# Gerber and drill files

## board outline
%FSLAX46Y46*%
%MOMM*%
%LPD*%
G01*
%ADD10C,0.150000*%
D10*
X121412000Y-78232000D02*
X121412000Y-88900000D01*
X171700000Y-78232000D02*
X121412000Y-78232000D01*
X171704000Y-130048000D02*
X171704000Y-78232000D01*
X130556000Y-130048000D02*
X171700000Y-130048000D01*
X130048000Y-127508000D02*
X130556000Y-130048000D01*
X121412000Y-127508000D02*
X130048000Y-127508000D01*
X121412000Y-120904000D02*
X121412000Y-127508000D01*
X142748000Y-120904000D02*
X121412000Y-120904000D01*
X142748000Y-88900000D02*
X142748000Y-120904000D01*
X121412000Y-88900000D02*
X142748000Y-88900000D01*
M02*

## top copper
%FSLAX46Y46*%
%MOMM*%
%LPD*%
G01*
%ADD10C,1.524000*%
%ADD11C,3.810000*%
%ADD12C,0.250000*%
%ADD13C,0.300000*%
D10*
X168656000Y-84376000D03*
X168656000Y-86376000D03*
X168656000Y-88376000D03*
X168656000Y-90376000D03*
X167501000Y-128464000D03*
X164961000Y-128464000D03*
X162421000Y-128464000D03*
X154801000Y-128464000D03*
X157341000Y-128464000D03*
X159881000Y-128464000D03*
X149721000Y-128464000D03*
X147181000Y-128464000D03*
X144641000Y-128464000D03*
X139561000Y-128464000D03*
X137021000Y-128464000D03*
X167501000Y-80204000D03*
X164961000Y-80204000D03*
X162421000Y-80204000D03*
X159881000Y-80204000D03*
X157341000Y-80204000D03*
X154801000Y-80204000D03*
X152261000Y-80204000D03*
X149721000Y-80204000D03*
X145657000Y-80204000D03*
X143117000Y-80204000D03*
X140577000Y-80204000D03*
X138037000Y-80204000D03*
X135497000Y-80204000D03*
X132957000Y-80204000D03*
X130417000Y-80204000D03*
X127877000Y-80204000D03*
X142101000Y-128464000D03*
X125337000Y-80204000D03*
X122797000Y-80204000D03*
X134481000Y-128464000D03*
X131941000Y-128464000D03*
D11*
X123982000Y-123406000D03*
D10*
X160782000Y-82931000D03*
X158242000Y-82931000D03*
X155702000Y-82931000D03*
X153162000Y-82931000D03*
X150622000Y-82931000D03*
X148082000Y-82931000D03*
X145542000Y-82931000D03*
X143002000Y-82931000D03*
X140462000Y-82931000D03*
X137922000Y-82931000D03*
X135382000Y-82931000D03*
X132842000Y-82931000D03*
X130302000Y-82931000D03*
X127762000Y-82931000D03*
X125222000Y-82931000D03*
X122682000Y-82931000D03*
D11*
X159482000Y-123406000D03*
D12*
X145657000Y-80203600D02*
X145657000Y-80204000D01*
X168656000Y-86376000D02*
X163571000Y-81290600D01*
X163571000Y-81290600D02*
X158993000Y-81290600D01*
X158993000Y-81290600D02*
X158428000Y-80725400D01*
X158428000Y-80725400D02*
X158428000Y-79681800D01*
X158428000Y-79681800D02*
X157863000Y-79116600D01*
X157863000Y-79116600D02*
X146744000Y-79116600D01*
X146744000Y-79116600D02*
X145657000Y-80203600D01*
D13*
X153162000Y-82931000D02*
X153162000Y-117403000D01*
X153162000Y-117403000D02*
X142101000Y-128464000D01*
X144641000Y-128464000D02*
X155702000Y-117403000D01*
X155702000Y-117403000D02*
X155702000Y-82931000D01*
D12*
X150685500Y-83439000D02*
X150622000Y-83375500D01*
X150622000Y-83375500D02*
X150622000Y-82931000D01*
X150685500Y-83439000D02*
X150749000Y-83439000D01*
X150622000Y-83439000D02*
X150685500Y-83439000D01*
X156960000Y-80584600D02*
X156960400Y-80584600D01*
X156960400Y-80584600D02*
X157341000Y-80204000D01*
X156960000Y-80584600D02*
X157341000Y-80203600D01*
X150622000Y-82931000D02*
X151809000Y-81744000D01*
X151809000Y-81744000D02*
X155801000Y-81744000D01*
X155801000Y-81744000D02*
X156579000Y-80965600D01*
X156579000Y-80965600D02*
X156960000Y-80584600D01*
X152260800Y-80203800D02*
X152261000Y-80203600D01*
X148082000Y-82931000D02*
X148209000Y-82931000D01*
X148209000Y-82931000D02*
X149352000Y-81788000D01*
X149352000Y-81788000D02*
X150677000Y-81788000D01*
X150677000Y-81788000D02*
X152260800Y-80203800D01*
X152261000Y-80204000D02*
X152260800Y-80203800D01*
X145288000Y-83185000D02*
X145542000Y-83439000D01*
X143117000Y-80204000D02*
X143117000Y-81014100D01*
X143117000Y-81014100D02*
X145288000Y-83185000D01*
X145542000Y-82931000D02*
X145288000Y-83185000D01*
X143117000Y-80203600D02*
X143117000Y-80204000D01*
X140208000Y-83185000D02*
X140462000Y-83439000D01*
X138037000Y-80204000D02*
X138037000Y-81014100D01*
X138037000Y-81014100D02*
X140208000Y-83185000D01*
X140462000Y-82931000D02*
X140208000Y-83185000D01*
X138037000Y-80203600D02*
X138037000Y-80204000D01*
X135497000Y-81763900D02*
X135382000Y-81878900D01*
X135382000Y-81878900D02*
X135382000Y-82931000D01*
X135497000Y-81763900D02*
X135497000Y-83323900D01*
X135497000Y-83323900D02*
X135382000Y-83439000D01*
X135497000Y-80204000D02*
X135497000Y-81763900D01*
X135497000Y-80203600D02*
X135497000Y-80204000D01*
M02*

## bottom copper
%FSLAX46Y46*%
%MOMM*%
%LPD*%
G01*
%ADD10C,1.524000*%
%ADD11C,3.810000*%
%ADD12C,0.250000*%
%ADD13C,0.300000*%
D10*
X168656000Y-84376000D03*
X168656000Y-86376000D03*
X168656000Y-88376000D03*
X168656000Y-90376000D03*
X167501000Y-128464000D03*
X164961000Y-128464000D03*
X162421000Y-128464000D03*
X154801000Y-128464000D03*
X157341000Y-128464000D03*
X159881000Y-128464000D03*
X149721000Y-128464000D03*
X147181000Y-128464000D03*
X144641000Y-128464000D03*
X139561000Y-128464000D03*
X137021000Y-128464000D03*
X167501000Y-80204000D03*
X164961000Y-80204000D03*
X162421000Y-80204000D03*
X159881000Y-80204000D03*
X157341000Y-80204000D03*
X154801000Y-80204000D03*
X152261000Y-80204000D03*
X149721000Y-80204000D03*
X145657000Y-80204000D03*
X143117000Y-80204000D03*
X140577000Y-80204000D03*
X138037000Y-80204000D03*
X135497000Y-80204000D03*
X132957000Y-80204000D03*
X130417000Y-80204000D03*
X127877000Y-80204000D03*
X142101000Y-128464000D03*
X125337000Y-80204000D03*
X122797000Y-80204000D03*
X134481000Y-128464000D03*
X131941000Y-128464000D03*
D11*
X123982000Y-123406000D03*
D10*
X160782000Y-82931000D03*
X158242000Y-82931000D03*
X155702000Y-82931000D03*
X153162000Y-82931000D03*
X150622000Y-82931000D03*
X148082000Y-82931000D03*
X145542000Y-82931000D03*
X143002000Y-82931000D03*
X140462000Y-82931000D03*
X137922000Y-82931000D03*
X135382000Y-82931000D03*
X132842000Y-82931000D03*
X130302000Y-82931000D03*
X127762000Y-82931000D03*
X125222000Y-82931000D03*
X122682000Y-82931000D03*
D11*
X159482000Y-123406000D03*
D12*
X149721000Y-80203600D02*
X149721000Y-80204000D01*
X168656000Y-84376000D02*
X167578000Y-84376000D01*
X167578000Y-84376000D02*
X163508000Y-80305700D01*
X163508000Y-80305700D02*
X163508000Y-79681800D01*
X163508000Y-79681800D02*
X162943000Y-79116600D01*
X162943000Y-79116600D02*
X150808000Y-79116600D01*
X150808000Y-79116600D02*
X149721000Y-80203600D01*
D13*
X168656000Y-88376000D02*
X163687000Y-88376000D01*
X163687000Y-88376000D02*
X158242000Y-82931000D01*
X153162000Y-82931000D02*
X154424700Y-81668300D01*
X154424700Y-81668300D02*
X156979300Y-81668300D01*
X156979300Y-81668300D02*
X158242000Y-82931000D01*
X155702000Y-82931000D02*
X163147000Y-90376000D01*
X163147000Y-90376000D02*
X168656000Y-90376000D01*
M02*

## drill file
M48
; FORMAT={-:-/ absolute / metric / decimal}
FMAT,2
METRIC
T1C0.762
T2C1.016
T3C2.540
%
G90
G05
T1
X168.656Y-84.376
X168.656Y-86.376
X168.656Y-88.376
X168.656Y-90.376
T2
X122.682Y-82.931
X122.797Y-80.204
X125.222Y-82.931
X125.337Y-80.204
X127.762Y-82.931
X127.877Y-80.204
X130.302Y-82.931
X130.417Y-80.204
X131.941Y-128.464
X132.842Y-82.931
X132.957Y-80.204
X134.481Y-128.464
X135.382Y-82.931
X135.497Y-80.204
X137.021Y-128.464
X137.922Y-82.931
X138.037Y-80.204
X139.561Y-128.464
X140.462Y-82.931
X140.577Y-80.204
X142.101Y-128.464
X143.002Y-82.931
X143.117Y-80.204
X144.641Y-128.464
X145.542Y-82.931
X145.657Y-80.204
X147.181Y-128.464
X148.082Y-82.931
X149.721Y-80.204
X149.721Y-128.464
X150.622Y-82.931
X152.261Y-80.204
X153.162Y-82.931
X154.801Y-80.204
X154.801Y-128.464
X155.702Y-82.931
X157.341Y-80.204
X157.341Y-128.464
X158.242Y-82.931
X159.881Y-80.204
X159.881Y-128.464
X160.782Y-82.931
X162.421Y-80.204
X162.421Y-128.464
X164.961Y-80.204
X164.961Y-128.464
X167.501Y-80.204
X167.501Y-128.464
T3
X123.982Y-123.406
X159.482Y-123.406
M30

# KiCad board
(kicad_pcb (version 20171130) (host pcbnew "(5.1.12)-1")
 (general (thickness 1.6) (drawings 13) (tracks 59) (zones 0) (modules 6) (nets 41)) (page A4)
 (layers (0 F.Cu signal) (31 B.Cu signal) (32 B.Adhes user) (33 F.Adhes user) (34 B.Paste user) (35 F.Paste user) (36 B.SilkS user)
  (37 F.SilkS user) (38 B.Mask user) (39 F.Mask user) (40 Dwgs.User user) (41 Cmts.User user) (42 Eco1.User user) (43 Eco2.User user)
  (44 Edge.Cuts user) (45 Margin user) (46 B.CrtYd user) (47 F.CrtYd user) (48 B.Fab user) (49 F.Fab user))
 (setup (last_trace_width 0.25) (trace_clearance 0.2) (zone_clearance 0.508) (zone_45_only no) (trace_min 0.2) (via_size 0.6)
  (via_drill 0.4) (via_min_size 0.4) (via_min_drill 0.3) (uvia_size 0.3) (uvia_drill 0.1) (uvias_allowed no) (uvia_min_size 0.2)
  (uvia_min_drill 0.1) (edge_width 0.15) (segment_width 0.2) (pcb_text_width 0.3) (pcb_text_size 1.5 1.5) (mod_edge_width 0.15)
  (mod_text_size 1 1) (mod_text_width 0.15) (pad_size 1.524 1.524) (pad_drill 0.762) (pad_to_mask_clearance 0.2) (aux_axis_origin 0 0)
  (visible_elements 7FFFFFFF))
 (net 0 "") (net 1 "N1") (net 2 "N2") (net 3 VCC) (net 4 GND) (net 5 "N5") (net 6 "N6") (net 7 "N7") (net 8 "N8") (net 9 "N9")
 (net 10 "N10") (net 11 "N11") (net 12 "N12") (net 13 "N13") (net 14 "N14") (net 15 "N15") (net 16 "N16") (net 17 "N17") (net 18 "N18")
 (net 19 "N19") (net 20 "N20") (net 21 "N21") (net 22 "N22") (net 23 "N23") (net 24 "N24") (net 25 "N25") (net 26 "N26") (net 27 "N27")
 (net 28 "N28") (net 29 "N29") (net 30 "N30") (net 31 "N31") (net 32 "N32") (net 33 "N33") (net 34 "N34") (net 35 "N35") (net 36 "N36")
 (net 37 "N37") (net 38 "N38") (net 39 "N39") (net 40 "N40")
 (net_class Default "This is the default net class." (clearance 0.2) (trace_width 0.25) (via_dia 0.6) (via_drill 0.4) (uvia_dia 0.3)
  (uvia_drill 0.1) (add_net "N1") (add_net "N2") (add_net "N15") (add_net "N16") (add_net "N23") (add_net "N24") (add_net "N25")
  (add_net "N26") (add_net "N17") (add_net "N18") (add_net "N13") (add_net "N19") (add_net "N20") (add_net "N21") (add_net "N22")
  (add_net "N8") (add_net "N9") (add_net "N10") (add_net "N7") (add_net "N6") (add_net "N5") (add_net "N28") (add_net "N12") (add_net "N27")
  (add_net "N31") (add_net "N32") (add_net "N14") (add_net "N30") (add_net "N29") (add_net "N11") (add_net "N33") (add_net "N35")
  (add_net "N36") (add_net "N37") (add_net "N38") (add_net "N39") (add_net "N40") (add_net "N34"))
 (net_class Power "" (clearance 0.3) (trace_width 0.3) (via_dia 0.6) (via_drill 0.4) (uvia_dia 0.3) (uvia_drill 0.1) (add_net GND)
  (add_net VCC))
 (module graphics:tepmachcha (layer B.Cu) (at 166.624 113.665 90)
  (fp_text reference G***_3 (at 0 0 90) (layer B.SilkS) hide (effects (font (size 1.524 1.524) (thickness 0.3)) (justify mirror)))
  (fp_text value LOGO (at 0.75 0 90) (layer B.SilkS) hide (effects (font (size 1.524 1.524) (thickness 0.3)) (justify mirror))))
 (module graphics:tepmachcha (layer F.Cu) (at 167.386 100.33 270)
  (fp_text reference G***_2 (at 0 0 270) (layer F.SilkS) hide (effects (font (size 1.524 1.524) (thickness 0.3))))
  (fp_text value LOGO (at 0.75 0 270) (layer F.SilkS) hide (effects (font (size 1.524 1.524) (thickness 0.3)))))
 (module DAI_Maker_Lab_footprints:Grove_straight (layer F.Cu) (at 168.656 87.376 270)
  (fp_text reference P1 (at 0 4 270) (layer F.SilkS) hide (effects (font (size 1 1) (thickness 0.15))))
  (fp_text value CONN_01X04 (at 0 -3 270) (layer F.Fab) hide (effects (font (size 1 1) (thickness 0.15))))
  (pad 1 thru_hole circle (at -3 0 270) (size 1.524 1.524) (drill 0.762) (layers *.Cu *.Mask F.SilkS) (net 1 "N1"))
  (pad 2 thru_hole circle (at -1 0 270) (size 1.524 1.524) (drill 0.762) (layers *.Cu *.Mask F.SilkS) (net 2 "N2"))
  (pad 3 thru_hole circle (at 1 0 270) (size 1.524 1.524) (drill 0.762) (layers *.Cu *.Mask F.SilkS) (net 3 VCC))
  (pad 4 thru_hole circle (at 3 0 270) (size 1.524 1.524) (drill 0.762) (layers *.Cu *.Mask F.SilkS) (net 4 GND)))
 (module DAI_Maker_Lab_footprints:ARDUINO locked (layer F.Cu) (at 148.501 105.004)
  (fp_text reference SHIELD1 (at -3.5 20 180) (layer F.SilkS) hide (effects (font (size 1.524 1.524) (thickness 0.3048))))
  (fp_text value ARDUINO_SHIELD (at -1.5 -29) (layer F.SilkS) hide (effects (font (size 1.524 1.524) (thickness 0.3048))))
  (pad AD5 thru_hole circle (at 19 23.46 90) (size 1.524 1.524) (drill 1.016) (layers *.Cu *.Mask F.SilkS) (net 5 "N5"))
  (pad AD4 thru_hole circle (at 16.46 23.46 90) (size 1.524 1.524) (drill 1.016) (layers *.Cu *.Mask F.SilkS) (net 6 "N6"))
  (pad AD3 thru_hole circle (at 13.92 23.46 90) (size 1.524 1.524) (drill 1.016) (layers *.Cu *.Mask F.SilkS) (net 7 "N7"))
  (pad AD0 thru_hole circle (at 6.3 23.46 90) (size 1.524 1.524) (drill 1.016) (layers *.Cu *.Mask F.SilkS) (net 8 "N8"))
  (pad AD1 thru_hole circle (at 8.84 23.46 90) (size 1.524 1.524) (drill 1.016) (layers *.Cu *.Mask F.SilkS) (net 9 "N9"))
  (pad AD2 thru_hole circle (at 11.38 23.46 90) (size 1.524 1.524) (drill 1.016) (layers *.Cu *.Mask F.SilkS) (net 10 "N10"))
  (pad V_IN thru_hole circle (at 1.22 23.46 90) (size 1.524 1.524) (drill 1.016) (layers *.Cu *.Mask F.SilkS) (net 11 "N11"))
  (pad GND2 thru_hole circle (at -1.32 23.46 90) (size 1.524 1.524) (drill 1.016) (layers *.Cu *.Mask F.SilkS) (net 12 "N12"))
  (pad GND1 thru_hole circle (at -3.86 23.46 90) (size 1.524 1.524) (drill 1.016) (layers *.Cu *.Mask F.SilkS) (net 4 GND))
  (pad 3V3 thru_hole circle (at -8.94 23.46 90) (size 1.524 1.524) (drill 1.016) (layers *.Cu *.Mask F.SilkS) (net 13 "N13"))
  (pad RST thru_hole circle (at -11.48 23.46 90) (size 1.524 1.524) (drill 1.016) (layers *.Cu *.Mask F.SilkS) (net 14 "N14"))
  (pad 0 thru_hole circle (at 19 -24.8 90) (size 1.524 1.524) (drill 1.016) (layers *.Cu *.Mask F.SilkS) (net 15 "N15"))
  (pad 1 thru_hole circle (at 16.46 -24.8 90) (size 1.524 1.524) (drill 1.016) (layers *.Cu *.Mask F.SilkS) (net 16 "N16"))
  (pad 2 thru_hole circle (at 13.92 -24.8 90) (size 1.524 1.524) (drill 1.016) (layers *.Cu *.Mask F.SilkS) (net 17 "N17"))
  (pad 3 thru_hole circle (at 11.38 -24.8 90) (size 1.524 1.524) (drill 1.016) (layers *.Cu *.Mask F.SilkS) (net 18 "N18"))
  (pad 4 thru_hole circle (at 8.84 -24.8 90) (size 1.524 1.524) (drill 1.016) (layers *.Cu *.Mask F.SilkS) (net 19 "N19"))
  (pad 5 thru_hole circle (at 6.3 -24.8 90) (size 1.524 1.524) (drill 1.016) (layers *.Cu *.Mask F.SilkS) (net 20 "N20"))
  (pad 6 thru_hole circle (at 3.76 -24.8 90) (size 1.524 1.524) (drill 1.016) (layers *.Cu *.Mask F.SilkS) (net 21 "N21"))
  (pad 7 thru_hole circle (at 1.22 -24.8 90) (size 1.524 1.524) (drill 1.016) (layers *.Cu *.Mask F.SilkS) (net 1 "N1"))
  (pad 8 thru_hole circle (at -2.844 -24.8 90) (size 1.524 1.524) (drill 1.016) (layers *.Cu *.Mask F.SilkS) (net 2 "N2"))
  (pad 9 thru_hole circle (at -5.384 -24.8 90) (size 1.524 1.524) (drill 1.016) (layers *.Cu *.Mask F.SilkS) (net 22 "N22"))
  (pad 10 thru_hole circle (at -7.924 -24.8 90) (size 1.524 1.524) (drill 1.016) (layers *.Cu *.Mask F.SilkS) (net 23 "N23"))
  (pad 11 thru_hole circle (at -10.464 -24.8 90) (size 1.524 1.524) (drill 1.016) (layers *.Cu *.Mask F.SilkS) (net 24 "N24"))
  (pad 12 thru_hole circle (at -13.004 -24.8 90) (size 1.524 1.524) (drill 1.016) (layers *.Cu *.Mask F.SilkS) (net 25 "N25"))
  (pad 13 thru_hole circle (at -15.544 -24.8 90) (size 1.524 1.524) (drill 1.016) (layers *.Cu *.Mask F.SilkS) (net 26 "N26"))
  (pad GND3 thru_hole circle (at -18.084 -24.8 90) (size 1.524 1.524) (drill 1.016) (layers *.Cu *.Mask F.SilkS) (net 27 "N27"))
  (pad AREF thru_hole circle (at -20.624 -24.8 90) (size 1.524 1.524) (drill 1.016) (layers *.Cu *.Mask F.SilkS) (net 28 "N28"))
  (pad 5V thru_hole circle (at -6.4 23.46 90) (size 1.524 1.524) (drill 1.016) (layers *.Cu *.Mask F.SilkS) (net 3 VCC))
  (pad SDA thru_hole circle (at -23.164 -24.8 90) (size 1.524 1.524) (drill 1.016) (layers *.Cu *.Mask F.SilkS) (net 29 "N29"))
  (pad SCL thru_hole circle (at -25.704 -24.8 90) (size 1.524 1.524) (drill 1.016) (layers *.Cu *.Mask F.SilkS) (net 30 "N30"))
  (pad IO_R thru_hole circle (at -14.02 23.46 90) (size 1.524 1.524) (drill 1.016) (layers *.Cu *.Mask F.SilkS) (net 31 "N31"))
  (pad NC thru_hole circle (at -16.56 23.46 90) (size 1.524 1.524) (drill 1.016) (layers *.Cu *.Mask F.SilkS) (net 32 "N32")))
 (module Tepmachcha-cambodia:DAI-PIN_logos (layer B.Cu) (at 155.829 103.505 90)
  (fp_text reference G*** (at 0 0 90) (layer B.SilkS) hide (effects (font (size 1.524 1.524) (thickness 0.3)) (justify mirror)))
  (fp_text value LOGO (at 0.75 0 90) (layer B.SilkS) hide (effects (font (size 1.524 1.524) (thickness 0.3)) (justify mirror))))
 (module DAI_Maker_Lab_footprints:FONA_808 (layer F.Cu) (at 141.732 105.156 180)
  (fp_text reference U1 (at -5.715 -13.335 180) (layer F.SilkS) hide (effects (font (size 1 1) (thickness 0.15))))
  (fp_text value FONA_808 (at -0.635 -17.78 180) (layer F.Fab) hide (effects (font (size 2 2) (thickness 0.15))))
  (pad 18 thru_hole circle (at 17.75 -18.25 180) (size 3.81 3.81) (drill 2.54) (layers *.Cu *.Mask F.SilkS))
  (pad 1 thru_hole circle (at -19.05 22.225 180) (size 1.524 1.524) (drill 1.016) (layers *.Cu *.Mask F.SilkS) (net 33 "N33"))
  (pad 2 thru_hole circle (at -16.51 22.225 180) (size 1.524 1.524) (drill 1.016) (layers *.Cu *.Mask F.SilkS) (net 3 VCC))
  (pad 3 thru_hole circle (at -13.97 22.225 180) (size 1.524 1.524) (drill 1.016) (layers *.Cu *.Mask F.SilkS) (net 4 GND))
  (pad 4 thru_hole circle (at -11.43 22.225 180) (size 1.524 1.524) (drill 1.016) (layers *.Cu *.Mask F.SilkS) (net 3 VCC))
  (pad 5 thru_hole circle (at -8.89 22.225 180) (size 1.524 1.524) (drill 1.016) (layers *.Cu *.Mask F.SilkS) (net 19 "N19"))
  (pad 6 thru_hole circle (at -6.35 22.225 180) (size 1.524 1.524) (drill 1.016) (layers *.Cu *.Mask F.SilkS) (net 21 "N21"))
  (pad 7 thru_hole circle (at -3.81 22.225 180) (size 1.524 1.524) (drill 1.016) (layers *.Cu *.Mask F.SilkS) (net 22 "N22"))
  (pad 8 thru_hole circle (at -1.27 22.225 180) (size 1.524 1.524) (drill 1.016) (layers *.Cu *.Mask F.SilkS) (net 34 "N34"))
  (pad 9 thru_hole circle (at 1.27 22.225 180) (size 1.524 1.524) (drill 1.016) (layers *.Cu *.Mask F.SilkS) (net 24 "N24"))
  (pad 10 thru_hole circle (at 3.81 22.225 180) (size 1.524 1.524) (drill 1.016) (layers *.Cu *.Mask F.SilkS) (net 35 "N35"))
  (pad 11 thru_hole circle (at 6.35 22.225 180) (size 1.524 1.524) (drill 1.016) (layers *.Cu *.Mask F.SilkS) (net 25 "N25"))
  (pad 12 thru_hole circle (at 8.89 22.225 180) (size 1.524 1.524) (drill 1.016) (layers *.Cu *.Mask F.SilkS) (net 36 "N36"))
  (pad 13 thru_hole circle (at 11.43 22.225 180) (size 1.524 1.524) (drill 1.016) (layers *.Cu *.Mask F.SilkS) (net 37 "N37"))
  (pad 14 thru_hole circle (at 13.97 22.225 180) (size 1.524 1.524) (drill 1.016) (layers *.Cu *.Mask F.SilkS) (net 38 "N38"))
  (pad 15 thru_hole circle (at 16.51 22.225 180) (size 1.524 1.524) (drill 1.016) (layers *.Cu *.Mask F.SilkS) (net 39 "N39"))
  (pad 16 thru_hole circle (at 19.05 22.225 180) (size 1.524 1.524) (drill 1.016) (layers *.Cu *.Mask F.SilkS) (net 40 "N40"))
  (pad 17 thru_hole circle (at -17.75 -18.25 180) (size 3.81 3.81) (drill 2.54) (layers *.Cu *.Mask F.SilkS)))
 (gr_line (start 121.412 78.232) (end 121.412 88.9) (layer Edge.Cuts) (width 0.15))
 (gr_line (start 171.7 78.232) (end 121.412 78.232) (layer Edge.Cuts) (width 0.15))
 (gr_line (start 171.704 130.048) (end 171.704 78.232) (layer Edge.Cuts) (width 0.15))
 (gr_line (start 130.556 130.048) (end 171.7 130.048) (layer Edge.Cuts) (width 0.15))
 (gr_line (start 130.048 127.508) (end 130.556 130.048) (layer Edge.Cuts) (width 0.15))
 (gr_line (start 121.412 127.508) (end 130.048 127.508) (layer Edge.Cuts) (width 0.15))
 (gr_line (start 121.412 120.904) (end 121.412 127.508) (layer Edge.Cuts) (width 0.15))
 (gr_line (start 142.748 120.904) (end 121.412 120.904) (layer Edge.Cuts) (width 0.15))
 (gr_line (start 142.748 88.9) (end 142.748 120.904) (layer Edge.Cuts) (width 0.15))
 (gr_line (start 121.412 88.9) (end 142.748 88.9) (layer Edge.Cuts) (width 0.15))
 (segment (start 149.721 80.2036) (end 149.721 80.204) (width 0.25) (layer B.Cu) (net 1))
 (segment (start 168.656 84.376) (end 167.578 84.376) (width 0.25) (layer B.Cu) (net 1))
 (segment (start 167.578 84.376) (end 163.508 80.3057) (width 0.25) (layer B.Cu) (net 1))
 (segment (start 163.508 80.3057) (end 163.508 79.6818) (width 0.25) (layer B.Cu) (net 1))
 (segment (start 163.508 79.6818) (end 162.943 79.1166) (width 0.25) (layer B.Cu) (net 1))
 (segment (start 162.943 79.1166) (end 150.808 79.1166) (width 0.25) (layer B.Cu) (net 1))
 (segment (start 150.808 79.1166) (end 149.721 80.2036) (width 0.25) (layer B.Cu) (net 1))
 (segment (start 145.657 80.2036) (end 145.657 80.204) (width 0.25) (layer F.Cu) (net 2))
 (segment (start 168.656 86.376) (end 163.571 81.2906) (width 0.25) (layer F.Cu) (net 2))
 (segment (start 163.571 81.2906) (end 158.993 81.2906) (width 0.25) (layer F.Cu) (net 2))
 (segment (start 158.993 81.2906) (end 158.428 80.7254) (width 0.25) (layer F.Cu) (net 2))
 (segment (start 158.428 80.7254) (end 158.428 79.6818) (width 0.25) (layer F.Cu) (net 2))
 (segment (start 158.428 79.6818) (end 157.863 79.1166) (width 0.25) (layer F.Cu) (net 2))
 (segment (start 157.863 79.1166) (end 146.744 79.1166) (width 0.25) (layer F.Cu) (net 2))
 (segment (start 146.744 79.1166) (end 145.657 80.2036) (width 0.25) (layer F.Cu) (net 2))
 (segment (start 168.656 88.376) (end 163.687 88.376) (width 0.3) (layer B.Cu) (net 3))
 (segment (start 163.687 88.376) (end 158.242 82.931) (width 0.3) (layer B.Cu) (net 3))
 (segment (start 153.162 82.931) (end 153.162 117.403) (width 0.3) (layer F.Cu) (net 3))
 (segment (start 153.162 117.403) (end 142.101 128.464) (width 0.3) (layer F.Cu) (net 3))
 (segment (start 153.162 82.931) (end 154.4247 81.6683) (width 0.3) (layer B.Cu) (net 3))
 (segment (start 154.4247 81.6683) (end 156.9793 81.6683) (width 0.3) (layer B.Cu) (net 3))
 (segment (start 156.9793 81.6683) (end 158.242 82.931) (width 0.3) (layer B.Cu) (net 3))
 (segment (start 144.641 128.464) (end 155.702 117.403) (width 0.3) (layer F.Cu) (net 4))
 (segment (start 155.702 117.403) (end 155.702 82.931) (width 0.3) (layer F.Cu) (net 4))
 (segment (start 155.702 82.931) (end 163.147 90.376) (width 0.3) (layer B.Cu) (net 4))
 (segment (start 163.147 90.376) (end 168.656 90.376) (width 0.3) (layer B.Cu) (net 4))
 (segment (start 150.6855 83.439) (end 150.622 83.3755) (width 0.25) (layer F.Cu) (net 19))
 (segment (start 150.622 83.3755) (end 150.622 82.931) (width 0.25) (layer F.Cu) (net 19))
 (segment (start 150.6855 83.439) (end 150.749 83.439) (width 0.25) (layer F.Cu) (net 19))
 (segment (start 150.622 83.439) (end 150.6855 83.439) (width 0.25) (layer F.Cu) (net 19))
 (segment (start 156.96 80.5846) (end 156.9604 80.5846) (width 0.25) (layer F.Cu) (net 19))
 (segment (start 156.9604 80.5846) (end 157.341 80.204) (width 0.25) (layer F.Cu) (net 19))
 (segment (start 156.96 80.5846) (end 157.341 80.2036) (width 0.25) (layer F.Cu) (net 19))
 (segment (start 150.622 82.931) (end 151.809 81.744) (width 0.25) (layer F.Cu) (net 19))
 (segment (start 151.809 81.744) (end 155.801 81.744) (width 0.25) (layer F.Cu) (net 19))
 (segment (start 155.801 81.744) (end 156.579 80.9656) (width 0.25) (layer F.Cu) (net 19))
 (segment (start 156.579 80.9656) (end 156.96 80.5846) (width 0.25) (layer F.Cu) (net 19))
 (segment (start 152.2608 80.2038) (end 152.261 80.2036) (width 0.25) (layer F.Cu) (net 21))
 (segment (start 148.082 82.931) (end 148.209 82.931) (width 0.25) (layer F.Cu) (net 21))
 (segment (start 148.209 82.931) (end 149.352 81.788) (width 0.25) (layer F.Cu) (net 21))
 (segment (start 149.352 81.788) (end 150.677 81.788) (width 0.25) (layer F.Cu) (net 21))
 (segment (start 150.677 81.788) (end 152.2608 80.2038) (width 0.25) (layer F.Cu) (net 21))
 (segment (start 152.261 80.204) (end 152.2608 80.2038) (width 0.25) (layer F.Cu) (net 21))
 (segment (start 145.288 83.185) (end 145.542 83.439) (width 0.25) (layer F.Cu) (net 22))
 (segment (start 143.117 80.204) (end 143.117 81.0141) (width 0.25) (layer F.Cu) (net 22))
 (segment (start 143.117 81.0141) (end 145.288 83.185) (width 0.25) (layer F.Cu) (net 22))
 (segment (start 145.542 82.931) (end 145.288 83.185) (width 0.25) (layer F.Cu) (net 22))
 (segment (start 143.117 80.2036) (end 143.117 80.204) (width 0.25) (layer F.Cu) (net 22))
 (segment (start 140.208 83.185) (end 140.462 83.439) (width 0.25) (layer F.Cu) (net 24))
 (segment (start 138.037 80.204) (end 138.037 81.0141) (width 0.25) (layer F.Cu) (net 24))
 (segment (start 138.037 81.0141) (end 140.208 83.185) (width 0.25) (layer F.Cu) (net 24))
 (segment (start 140.462 82.931) (end 140.208 83.185) (width 0.25) (layer F.Cu) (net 24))
 (segment (start 138.037 80.2036) (end 138.037 80.204) (width 0.25) (layer F.Cu) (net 24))
 (segment (start 135.497 81.7639) (end 135.382 81.8789) (width 0.25) (layer F.Cu) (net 25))
 (segment (start 135.382 81.8789) (end 135.382 82.931) (width 0.25) (layer F.Cu) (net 25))
 (segment (start 135.497 81.7639) (end 135.497 83.3239) (width 0.25) (layer F.Cu) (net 25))
 (segment (start 135.497 83.3239) (end 135.382 83.439) (width 0.25) (layer F.Cu) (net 25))
 (segment (start 135.497 80.204) (end 135.497 81.7639) (width 0.25) (layer F.Cu) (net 25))
 (segment (start 135.497 80.2036) (end 135.497 80.204) (width 0.25) (layer F.Cu) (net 25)))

